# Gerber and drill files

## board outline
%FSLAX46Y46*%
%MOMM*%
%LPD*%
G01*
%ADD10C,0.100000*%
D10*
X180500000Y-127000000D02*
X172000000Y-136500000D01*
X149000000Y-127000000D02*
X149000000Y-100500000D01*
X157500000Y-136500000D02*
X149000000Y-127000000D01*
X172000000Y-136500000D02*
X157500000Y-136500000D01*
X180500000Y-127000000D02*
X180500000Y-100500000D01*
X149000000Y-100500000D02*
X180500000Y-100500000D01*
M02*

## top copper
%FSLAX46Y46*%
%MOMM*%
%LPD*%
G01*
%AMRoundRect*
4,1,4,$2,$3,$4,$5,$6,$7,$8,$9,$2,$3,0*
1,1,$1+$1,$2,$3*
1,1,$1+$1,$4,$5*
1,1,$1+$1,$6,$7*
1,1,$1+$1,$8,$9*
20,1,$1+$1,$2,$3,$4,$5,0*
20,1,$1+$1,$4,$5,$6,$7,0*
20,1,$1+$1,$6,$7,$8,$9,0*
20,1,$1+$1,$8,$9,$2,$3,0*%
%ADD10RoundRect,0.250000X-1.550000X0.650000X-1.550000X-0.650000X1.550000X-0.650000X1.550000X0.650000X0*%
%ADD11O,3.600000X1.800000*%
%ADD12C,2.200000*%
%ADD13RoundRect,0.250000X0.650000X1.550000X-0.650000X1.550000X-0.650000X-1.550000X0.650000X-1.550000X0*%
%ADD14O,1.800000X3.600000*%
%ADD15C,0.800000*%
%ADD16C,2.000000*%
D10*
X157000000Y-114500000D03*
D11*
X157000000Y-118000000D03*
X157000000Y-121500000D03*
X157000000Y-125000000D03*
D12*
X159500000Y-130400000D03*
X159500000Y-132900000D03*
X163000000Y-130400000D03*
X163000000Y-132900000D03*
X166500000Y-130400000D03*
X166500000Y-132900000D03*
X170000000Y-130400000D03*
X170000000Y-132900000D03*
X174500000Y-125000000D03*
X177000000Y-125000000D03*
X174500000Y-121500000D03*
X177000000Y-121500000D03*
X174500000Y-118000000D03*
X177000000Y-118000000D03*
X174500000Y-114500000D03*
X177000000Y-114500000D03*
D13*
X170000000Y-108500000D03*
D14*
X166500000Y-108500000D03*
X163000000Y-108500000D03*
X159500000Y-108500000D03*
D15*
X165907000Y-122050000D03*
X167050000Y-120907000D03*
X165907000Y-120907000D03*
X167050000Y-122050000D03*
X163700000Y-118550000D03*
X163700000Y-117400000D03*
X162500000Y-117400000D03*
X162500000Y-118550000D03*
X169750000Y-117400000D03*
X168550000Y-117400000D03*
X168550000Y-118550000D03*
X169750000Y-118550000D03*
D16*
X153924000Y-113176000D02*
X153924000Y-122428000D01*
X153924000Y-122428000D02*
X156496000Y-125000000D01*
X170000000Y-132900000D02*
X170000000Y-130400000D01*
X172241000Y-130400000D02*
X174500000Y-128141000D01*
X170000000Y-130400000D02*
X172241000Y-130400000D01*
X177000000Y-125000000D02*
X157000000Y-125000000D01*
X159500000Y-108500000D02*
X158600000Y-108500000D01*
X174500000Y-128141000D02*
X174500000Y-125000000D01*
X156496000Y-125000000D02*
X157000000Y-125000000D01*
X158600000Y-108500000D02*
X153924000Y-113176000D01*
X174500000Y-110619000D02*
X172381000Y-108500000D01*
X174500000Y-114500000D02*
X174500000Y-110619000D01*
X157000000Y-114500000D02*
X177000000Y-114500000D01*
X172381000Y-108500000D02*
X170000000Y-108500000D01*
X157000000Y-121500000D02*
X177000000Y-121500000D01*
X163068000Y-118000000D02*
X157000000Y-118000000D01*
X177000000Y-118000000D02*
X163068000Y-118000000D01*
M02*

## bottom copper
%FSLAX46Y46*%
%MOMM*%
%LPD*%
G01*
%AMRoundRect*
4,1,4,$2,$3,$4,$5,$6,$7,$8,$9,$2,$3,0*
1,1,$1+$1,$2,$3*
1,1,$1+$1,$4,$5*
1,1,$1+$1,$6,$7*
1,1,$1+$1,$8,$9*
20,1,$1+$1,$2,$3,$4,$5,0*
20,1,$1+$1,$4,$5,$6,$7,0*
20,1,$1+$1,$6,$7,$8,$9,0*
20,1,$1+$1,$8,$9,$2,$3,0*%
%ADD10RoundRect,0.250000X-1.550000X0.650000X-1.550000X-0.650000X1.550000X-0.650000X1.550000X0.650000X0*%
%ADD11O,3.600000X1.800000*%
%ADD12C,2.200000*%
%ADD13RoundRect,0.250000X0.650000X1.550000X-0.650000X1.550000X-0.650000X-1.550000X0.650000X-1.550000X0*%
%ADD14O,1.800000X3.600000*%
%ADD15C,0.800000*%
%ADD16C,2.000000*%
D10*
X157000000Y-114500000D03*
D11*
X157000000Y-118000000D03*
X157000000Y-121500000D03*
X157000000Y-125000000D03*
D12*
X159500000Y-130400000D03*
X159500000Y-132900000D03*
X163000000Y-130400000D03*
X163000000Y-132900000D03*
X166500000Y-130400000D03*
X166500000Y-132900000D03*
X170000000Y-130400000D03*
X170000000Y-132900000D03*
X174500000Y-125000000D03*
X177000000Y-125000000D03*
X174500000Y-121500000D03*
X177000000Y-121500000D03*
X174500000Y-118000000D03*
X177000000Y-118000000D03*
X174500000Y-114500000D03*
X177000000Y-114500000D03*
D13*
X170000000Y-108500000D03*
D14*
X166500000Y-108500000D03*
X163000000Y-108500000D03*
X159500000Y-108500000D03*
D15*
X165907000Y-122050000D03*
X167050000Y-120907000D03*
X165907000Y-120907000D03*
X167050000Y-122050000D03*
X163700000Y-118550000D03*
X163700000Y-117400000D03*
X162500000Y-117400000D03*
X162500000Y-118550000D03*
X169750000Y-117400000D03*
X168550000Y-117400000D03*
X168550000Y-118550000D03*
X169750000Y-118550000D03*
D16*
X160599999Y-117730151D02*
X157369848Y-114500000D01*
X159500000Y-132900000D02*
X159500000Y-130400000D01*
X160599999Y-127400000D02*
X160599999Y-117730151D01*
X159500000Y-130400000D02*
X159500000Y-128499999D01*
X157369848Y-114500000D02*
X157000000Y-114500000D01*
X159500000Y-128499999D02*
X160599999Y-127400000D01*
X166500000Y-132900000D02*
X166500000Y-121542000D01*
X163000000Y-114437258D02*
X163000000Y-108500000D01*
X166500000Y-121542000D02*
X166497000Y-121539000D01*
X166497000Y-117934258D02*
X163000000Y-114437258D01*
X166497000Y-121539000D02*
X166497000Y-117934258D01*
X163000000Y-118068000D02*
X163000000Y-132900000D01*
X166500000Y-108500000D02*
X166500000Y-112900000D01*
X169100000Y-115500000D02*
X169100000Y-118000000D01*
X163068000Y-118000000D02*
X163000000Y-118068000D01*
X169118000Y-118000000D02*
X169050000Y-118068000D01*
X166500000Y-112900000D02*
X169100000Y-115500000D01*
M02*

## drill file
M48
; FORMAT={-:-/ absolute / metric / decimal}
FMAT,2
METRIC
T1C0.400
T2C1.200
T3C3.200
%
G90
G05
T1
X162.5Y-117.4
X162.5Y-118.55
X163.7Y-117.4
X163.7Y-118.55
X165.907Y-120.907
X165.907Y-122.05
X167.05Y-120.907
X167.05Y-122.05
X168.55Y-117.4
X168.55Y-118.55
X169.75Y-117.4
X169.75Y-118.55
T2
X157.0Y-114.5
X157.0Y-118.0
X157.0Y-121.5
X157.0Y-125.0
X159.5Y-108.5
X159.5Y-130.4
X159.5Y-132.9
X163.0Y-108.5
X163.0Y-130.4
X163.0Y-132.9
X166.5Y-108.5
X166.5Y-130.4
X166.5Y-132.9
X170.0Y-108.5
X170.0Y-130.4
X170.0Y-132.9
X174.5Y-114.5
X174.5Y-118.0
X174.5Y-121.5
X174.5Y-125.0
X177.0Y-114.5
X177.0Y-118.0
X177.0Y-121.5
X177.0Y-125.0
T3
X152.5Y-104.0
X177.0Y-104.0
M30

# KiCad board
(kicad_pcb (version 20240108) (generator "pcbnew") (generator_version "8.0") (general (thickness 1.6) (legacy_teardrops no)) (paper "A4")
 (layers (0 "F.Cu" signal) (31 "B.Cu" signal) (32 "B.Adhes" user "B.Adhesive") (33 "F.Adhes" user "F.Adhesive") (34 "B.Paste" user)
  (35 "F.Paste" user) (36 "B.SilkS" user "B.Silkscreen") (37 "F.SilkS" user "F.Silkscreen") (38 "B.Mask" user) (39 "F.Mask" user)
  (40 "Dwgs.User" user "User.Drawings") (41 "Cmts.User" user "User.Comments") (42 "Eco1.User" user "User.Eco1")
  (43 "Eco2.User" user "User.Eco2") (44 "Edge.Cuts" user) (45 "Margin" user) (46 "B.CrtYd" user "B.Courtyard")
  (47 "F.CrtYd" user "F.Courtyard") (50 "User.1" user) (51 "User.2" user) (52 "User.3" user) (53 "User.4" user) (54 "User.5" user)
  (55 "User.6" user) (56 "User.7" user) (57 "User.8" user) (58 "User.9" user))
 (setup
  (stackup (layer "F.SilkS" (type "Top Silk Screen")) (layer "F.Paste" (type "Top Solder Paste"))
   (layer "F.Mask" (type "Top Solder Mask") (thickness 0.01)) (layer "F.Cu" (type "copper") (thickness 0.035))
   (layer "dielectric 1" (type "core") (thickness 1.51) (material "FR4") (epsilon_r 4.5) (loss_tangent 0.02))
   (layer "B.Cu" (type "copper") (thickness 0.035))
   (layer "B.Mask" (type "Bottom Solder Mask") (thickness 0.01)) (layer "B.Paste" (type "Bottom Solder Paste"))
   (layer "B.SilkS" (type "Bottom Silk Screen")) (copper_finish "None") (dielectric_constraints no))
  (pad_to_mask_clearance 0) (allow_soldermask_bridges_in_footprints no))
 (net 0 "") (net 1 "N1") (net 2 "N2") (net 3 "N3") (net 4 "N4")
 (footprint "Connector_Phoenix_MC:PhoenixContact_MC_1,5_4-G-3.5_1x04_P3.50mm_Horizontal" (layer "F.Cu") (at 157 114.5 -90)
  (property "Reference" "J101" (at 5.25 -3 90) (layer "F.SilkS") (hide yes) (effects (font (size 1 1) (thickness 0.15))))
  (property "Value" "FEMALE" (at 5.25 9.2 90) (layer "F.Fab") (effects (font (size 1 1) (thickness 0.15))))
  (pad "1" thru_hole roundrect (at 0 0 270) (size 1.8 3.6) (drill 1.2) (layers "*.Cu" "*.Mask") (remove_unused_layers no)
   (roundrect_rratio 0.138889) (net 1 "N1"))
  (pad "2" thru_hole oval (at 3.5 0 270) (size 1.8 3.6) (drill 1.2) (layers "*.Cu" "*.Mask") (remove_unused_layers no) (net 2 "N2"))
  (pad "3" thru_hole oval (at 7 0 270) (size 1.8 3.6) (drill 1.2) (layers "*.Cu" "*.Mask") (remove_unused_layers no) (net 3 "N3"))
  (pad "4" thru_hole oval (at 10.5 0 270) (size 1.8 3.6) (drill 1.2) (layers "*.Cu" "*.Mask") (remove_unused_layers no) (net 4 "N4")))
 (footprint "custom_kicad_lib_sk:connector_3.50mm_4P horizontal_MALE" (layer "F.Cu") (at 164.75 130.4)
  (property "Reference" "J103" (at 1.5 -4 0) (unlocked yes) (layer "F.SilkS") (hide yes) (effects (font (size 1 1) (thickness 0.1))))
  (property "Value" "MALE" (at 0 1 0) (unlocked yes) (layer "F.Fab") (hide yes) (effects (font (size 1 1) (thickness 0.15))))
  (pad "1" thru_hole circle (at -5.25 0) (size 2.2 2.2) (drill 1.2) (layers "*.Cu" "*.Mask") (remove_unused_layers no) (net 1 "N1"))
  (pad "1" thru_hole circle (at -5.25 2.5) (size 2.2 2.2) (drill 1.2) (layers "*.Cu" "*.Mask") (remove_unused_layers no) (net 1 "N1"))
  (pad "2" thru_hole circle (at -1.75 0) (size 2.2 2.2) (drill 1.2) (layers "*.Cu" "*.Mask") (remove_unused_layers no) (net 2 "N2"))
  (pad "2" thru_hole circle (at -1.75 2.5) (size 2.2 2.2) (drill 1.2) (layers "*.Cu" "*.Mask") (remove_unused_layers no) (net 2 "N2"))
  (pad "3" thru_hole circle (at 1.75 0) (size 2.2 2.2) (drill 1.2) (layers "*.Cu" "*.Mask") (remove_unused_layers no) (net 3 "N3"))
  (pad "3" thru_hole circle (at 1.75 2.5) (size 2.2 2.2) (drill 1.2) (layers "*.Cu" "*.Mask") (remove_unused_layers no) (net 3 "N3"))
  (pad "4" thru_hole circle (at 5.25 0) (size 2.2 2.2) (drill 1.2) (layers "*.Cu" "*.Mask") (remove_unused_layers no) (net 4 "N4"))
  (pad "4" thru_hole circle (at 5.25 2.5) (size 2.2 2.2) (drill 1.2) (layers "*.Cu" "*.Mask") (remove_unused_layers no) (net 4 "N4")))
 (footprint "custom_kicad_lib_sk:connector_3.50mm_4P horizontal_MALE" (layer "F.Cu") (at 174.5 119.75 90)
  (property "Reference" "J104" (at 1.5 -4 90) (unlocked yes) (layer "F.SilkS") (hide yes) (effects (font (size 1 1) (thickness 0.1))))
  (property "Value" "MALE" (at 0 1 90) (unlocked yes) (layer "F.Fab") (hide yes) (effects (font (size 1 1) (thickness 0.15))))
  (pad "1" thru_hole circle (at -5.25 0 90) (size 2.2 2.2) (drill 1.2) (layers "*.Cu" "*.Mask") (remove_unused_layers no) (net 4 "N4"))
  (pad "1" thru_hole circle (at -5.25 2.5 90) (size 2.2 2.2) (drill 1.2) (layers "*.Cu" "*.Mask") (remove_unused_layers no) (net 4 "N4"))
  (pad "2" thru_hole circle (at -1.75 0 90) (size 2.2 2.2) (drill 1.2) (layers "*.Cu" "*.Mask") (remove_unused_layers no) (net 3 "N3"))
  (pad "2" thru_hole circle (at -1.75 2.5 90) (size 2.2 2.2) (drill 1.2) (layers "*.Cu" "*.Mask") (remove_unused_layers no) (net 3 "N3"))
  (pad "3" thru_hole circle (at 1.75 0 90) (size 2.2 2.2) (drill 1.2) (layers "*.Cu" "*.Mask") (remove_unused_layers no) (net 2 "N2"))
  (pad "3" thru_hole circle (at 1.75 2.5 90) (size 2.2 2.2) (drill 1.2) (layers "*.Cu" "*.Mask") (remove_unused_layers no) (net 2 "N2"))
  (pad "4" thru_hole circle (at 5.25 0 90) (size 2.2 2.2) (drill 1.2) (layers "*.Cu" "*.Mask") (remove_unused_layers no) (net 1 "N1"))
  (pad "4" thru_hole circle (at 5.25 2.5 90) (size 2.2 2.2) (drill 1.2) (layers "*.Cu" "*.Mask") (remove_unused_layers no) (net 1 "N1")))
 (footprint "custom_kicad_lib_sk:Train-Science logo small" (layer "F.Cu") (at 165.735 120.523)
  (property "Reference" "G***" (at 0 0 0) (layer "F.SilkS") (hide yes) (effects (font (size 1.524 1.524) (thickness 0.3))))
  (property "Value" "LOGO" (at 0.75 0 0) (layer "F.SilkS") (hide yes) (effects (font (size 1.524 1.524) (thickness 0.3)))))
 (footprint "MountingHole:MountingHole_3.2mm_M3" (layer "F.Cu") (at 152.5 104)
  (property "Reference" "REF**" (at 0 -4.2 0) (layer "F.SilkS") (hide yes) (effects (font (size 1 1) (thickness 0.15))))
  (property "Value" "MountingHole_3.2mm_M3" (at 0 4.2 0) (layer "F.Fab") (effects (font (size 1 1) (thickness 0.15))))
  (pad "" np_thru_hole circle (at 0 0) (size 3.2 3.2) (drill 3.2) (layers "*.Cu" "*.Mask")))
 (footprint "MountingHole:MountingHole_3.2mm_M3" (layer "F.Cu") (at 177 104)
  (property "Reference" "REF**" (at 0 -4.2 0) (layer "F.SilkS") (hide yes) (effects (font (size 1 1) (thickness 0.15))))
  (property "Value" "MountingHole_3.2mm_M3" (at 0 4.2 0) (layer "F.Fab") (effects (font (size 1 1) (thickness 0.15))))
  (pad "" np_thru_hole circle (at 0 0) (size 3.2 3.2) (drill 3.2) (layers "F&B.Cu" "*.Mask")))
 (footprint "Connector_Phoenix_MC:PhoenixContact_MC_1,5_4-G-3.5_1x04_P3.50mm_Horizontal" (layer "F.Cu") (at 170 108.5 180)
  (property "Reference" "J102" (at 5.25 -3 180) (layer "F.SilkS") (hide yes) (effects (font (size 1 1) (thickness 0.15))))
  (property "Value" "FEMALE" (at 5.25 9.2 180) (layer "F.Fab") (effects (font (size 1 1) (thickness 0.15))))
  (pad "1" thru_hole roundrect (at 0 0 180) (size 1.8 3.6) (drill 1.2) (layers "*.Cu" "*.Mask") (remove_unused_layers no)
   (roundrect_rratio 0.138889) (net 1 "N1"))
  (pad "2" thru_hole oval (at 3.5 0 180) (size 1.8 3.6) (drill 1.2) (layers "*.Cu" "*.Mask") (remove_unused_layers no) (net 2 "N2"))
  (pad "3" thru_hole oval (at 7 0 180) (size 1.8 3.6) (drill 1.2) (layers "*.Cu" "*.Mask") (remove_unused_layers no) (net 3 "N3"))
  (pad "4" thru_hole oval (at 10.5 0 180) (size 1.8 3.6) (drill 1.2) (layers "*.Cu" "*.Mask") (remove_unused_layers no) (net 4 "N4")))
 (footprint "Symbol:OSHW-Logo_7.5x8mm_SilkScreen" (layer "B.Cu") (at 164.973 118.491 180)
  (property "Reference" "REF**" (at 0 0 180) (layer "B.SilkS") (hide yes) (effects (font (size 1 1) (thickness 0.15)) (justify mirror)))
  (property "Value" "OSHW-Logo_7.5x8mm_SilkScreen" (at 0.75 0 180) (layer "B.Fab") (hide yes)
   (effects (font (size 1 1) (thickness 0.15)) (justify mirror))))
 (gr_line (start 180.5 127) (end 172 136.5) (stroke (width 0.1) (type default)) (layer "Edge.Cuts"))
 (gr_line (start 149 127) (end 149 100.5) (stroke (width 0.1) (type default)) (layer "Edge.Cuts"))
 (gr_line (start 157.5 136.5) (end 149 127) (stroke (width 0.1) (type default)) (layer "Edge.Cuts"))
 (gr_line (start 172 136.5) (end 157.5 136.5) (stroke (width 0.1) (type default)) (layer "Edge.Cuts"))
 (gr_line (start 180.5 127) (end 180.5 100.5) (stroke (width 0.1) (type default)) (layer "Edge.Cuts"))
 (gr_line (start 149 100.5) (end 180.5 100.5) (stroke (width 0.1) (type default)) (layer "Edge.Cuts"))
 (segment (start 153.924 113.176) (end 153.924 122.428) (width 2) (layer "F.Cu") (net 4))
 (segment (start 153.924 122.428) (end 156.496 125) (width 2) (layer "F.Cu") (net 4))
 (segment (start 170 132.9) (end 170 130.4) (width 2) (layer "F.Cu") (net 4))
 (segment (start 172.241 130.4) (end 174.5 128.141) (width 2) (layer "F.Cu") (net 4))
 (segment (start 170 130.4) (end 172.241 130.4) (width 2) (layer "F.Cu") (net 4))
 (segment (start 177 125) (end 157 125) (width 2) (layer "F.Cu") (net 4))
 (segment (start 159.5 108.5) (end 158.6 108.5) (width 2) (layer "F.Cu") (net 4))
 (segment (start 174.5 128.141) (end 174.5 125) (width 2) (layer "F.Cu") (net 4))
 (segment (start 156.496 125) (end 157 125) (width 2) (layer "F.Cu") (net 4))
 (segment (start 158.6 108.5) (end 153.924 113.176) (width 2) (layer "F.Cu") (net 4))
 (segment (start 174.5 110.619) (end 172.381 108.5) (width 2) (layer "F.Cu") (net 1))
 (segment (start 174.5 114.5) (end 174.5 110.619) (width 2) (layer "F.Cu") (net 1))
 (segment (start 157 114.5) (end 177 114.5) (width 2) (layer "F.Cu") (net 1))
 (segment (start 172.381 108.5) (end 170 108.5) (width 2) (layer "F.Cu") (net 1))
 (segment (start 160.599999 117.730151) (end 157.369848 114.5) (width 2) (layer "B.Cu") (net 1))
 (segment (start 159.5 132.9) (end 159.5 130.4) (width 2) (layer "B.Cu") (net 1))
 (segment (start 160.599999 127.4) (end 160.599999 117.730151) (width 2) (layer "B.Cu") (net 1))
 (segment (start 159.5 130.4) (end 159.5 128.499999) (width 2) (layer "B.Cu") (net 1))
 (segment (start 157.369848 114.5) (end 157 114.5) (width 2) (layer "B.Cu") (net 1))
 (segment (start 159.5 128.499999) (end 160.599999 127.4) (width 2) (layer "B.Cu") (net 1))
 (segment (start 157 121.5) (end 177 121.5) (width 2) (layer "F.Cu") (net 3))
 (via (at 165.907 122.05) (size 0.8) (drill 0.4) (layers "F.Cu" "B.Cu") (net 3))
 (via (at 167.05 120.907) (size 0.8) (drill 0.4) (layers "F.Cu" "B.Cu") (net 3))
 (via (at 165.907 120.907) (size 0.8) (drill 0.4) (layers "F.Cu" "B.Cu") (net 3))
 (via (at 167.05 122.05) (size 0.8) (drill 0.4) (layers "F.Cu" "B.Cu") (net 3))
 (segment (start 166.5 132.9) (end 166.5 121.542) (width 2) (layer "B.Cu") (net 3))
 (segment (start 163 114.437258) (end 163 108.5) (width 2) (layer "B.Cu") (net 3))
 (segment (start 166.5 121.542) (end 166.497 121.539) (width 2) (layer "B.Cu") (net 3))
 (segment (start 166.497 117.934258) (end 163 114.437258) (width 2) (layer "B.Cu") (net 3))
 (segment (start 166.497 121.539) (end 166.497 117.934258) (width 2) (layer "B.Cu") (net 3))
 (segment (start 163.068 118) (end 157 118) (width 2) (layer "F.Cu") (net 2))
 (segment (start 177 118) (end 163.068 118) (width 2) (layer "F.Cu") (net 2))
 (via (at 163.7 118.55) (size 0.8) (drill 0.4) (layers "F.Cu" "B.Cu") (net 2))
 (via (at 163.7 117.4) (size 0.8) (drill 0.4) (layers "F.Cu" "B.Cu") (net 2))
 (via (at 162.5 117.4) (size 0.8) (drill 0.4) (layers "F.Cu" "B.Cu") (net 2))
 (via (at 162.5 118.55) (size 0.8) (drill 0.4) (layers "F.Cu" "B.Cu") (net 2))
 (via (at 169.75 117.4) (size 0.8) (drill 0.4) (layers "F.Cu" "B.Cu") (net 2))
 (via (at 168.55 117.4) (size 0.8) (drill 0.4) (layers "F.Cu" "B.Cu") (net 2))
 (via (at 168.55 118.55) (size 0.8) (drill 0.4) (layers "F.Cu" "B.Cu") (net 2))
 (via (at 169.75 118.55) (size 0.8) (drill 0.4) (layers "F.Cu" "B.Cu") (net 2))
 (segment (start 163 118.068) (end 163 132.9) (width 2) (layer "B.Cu") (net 2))
 (segment (start 166.5 108.5) (end 166.5 112.9) (width 2) (layer "B.Cu") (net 2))
 (segment (start 169.1 115.5) (end 169.1 118) (width 2) (layer "B.Cu") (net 2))
 (segment (start 163.068 118) (end 163 118.068) (width 2) (layer "B.Cu") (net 2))
 (segment (start 169.118 118) (end 169.05 118.068) (width 2) (layer "B.Cu") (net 2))
 (segment (start 166.5 112.9) (end 169.1 115.5) (width 2) (layer "B.Cu") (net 2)))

